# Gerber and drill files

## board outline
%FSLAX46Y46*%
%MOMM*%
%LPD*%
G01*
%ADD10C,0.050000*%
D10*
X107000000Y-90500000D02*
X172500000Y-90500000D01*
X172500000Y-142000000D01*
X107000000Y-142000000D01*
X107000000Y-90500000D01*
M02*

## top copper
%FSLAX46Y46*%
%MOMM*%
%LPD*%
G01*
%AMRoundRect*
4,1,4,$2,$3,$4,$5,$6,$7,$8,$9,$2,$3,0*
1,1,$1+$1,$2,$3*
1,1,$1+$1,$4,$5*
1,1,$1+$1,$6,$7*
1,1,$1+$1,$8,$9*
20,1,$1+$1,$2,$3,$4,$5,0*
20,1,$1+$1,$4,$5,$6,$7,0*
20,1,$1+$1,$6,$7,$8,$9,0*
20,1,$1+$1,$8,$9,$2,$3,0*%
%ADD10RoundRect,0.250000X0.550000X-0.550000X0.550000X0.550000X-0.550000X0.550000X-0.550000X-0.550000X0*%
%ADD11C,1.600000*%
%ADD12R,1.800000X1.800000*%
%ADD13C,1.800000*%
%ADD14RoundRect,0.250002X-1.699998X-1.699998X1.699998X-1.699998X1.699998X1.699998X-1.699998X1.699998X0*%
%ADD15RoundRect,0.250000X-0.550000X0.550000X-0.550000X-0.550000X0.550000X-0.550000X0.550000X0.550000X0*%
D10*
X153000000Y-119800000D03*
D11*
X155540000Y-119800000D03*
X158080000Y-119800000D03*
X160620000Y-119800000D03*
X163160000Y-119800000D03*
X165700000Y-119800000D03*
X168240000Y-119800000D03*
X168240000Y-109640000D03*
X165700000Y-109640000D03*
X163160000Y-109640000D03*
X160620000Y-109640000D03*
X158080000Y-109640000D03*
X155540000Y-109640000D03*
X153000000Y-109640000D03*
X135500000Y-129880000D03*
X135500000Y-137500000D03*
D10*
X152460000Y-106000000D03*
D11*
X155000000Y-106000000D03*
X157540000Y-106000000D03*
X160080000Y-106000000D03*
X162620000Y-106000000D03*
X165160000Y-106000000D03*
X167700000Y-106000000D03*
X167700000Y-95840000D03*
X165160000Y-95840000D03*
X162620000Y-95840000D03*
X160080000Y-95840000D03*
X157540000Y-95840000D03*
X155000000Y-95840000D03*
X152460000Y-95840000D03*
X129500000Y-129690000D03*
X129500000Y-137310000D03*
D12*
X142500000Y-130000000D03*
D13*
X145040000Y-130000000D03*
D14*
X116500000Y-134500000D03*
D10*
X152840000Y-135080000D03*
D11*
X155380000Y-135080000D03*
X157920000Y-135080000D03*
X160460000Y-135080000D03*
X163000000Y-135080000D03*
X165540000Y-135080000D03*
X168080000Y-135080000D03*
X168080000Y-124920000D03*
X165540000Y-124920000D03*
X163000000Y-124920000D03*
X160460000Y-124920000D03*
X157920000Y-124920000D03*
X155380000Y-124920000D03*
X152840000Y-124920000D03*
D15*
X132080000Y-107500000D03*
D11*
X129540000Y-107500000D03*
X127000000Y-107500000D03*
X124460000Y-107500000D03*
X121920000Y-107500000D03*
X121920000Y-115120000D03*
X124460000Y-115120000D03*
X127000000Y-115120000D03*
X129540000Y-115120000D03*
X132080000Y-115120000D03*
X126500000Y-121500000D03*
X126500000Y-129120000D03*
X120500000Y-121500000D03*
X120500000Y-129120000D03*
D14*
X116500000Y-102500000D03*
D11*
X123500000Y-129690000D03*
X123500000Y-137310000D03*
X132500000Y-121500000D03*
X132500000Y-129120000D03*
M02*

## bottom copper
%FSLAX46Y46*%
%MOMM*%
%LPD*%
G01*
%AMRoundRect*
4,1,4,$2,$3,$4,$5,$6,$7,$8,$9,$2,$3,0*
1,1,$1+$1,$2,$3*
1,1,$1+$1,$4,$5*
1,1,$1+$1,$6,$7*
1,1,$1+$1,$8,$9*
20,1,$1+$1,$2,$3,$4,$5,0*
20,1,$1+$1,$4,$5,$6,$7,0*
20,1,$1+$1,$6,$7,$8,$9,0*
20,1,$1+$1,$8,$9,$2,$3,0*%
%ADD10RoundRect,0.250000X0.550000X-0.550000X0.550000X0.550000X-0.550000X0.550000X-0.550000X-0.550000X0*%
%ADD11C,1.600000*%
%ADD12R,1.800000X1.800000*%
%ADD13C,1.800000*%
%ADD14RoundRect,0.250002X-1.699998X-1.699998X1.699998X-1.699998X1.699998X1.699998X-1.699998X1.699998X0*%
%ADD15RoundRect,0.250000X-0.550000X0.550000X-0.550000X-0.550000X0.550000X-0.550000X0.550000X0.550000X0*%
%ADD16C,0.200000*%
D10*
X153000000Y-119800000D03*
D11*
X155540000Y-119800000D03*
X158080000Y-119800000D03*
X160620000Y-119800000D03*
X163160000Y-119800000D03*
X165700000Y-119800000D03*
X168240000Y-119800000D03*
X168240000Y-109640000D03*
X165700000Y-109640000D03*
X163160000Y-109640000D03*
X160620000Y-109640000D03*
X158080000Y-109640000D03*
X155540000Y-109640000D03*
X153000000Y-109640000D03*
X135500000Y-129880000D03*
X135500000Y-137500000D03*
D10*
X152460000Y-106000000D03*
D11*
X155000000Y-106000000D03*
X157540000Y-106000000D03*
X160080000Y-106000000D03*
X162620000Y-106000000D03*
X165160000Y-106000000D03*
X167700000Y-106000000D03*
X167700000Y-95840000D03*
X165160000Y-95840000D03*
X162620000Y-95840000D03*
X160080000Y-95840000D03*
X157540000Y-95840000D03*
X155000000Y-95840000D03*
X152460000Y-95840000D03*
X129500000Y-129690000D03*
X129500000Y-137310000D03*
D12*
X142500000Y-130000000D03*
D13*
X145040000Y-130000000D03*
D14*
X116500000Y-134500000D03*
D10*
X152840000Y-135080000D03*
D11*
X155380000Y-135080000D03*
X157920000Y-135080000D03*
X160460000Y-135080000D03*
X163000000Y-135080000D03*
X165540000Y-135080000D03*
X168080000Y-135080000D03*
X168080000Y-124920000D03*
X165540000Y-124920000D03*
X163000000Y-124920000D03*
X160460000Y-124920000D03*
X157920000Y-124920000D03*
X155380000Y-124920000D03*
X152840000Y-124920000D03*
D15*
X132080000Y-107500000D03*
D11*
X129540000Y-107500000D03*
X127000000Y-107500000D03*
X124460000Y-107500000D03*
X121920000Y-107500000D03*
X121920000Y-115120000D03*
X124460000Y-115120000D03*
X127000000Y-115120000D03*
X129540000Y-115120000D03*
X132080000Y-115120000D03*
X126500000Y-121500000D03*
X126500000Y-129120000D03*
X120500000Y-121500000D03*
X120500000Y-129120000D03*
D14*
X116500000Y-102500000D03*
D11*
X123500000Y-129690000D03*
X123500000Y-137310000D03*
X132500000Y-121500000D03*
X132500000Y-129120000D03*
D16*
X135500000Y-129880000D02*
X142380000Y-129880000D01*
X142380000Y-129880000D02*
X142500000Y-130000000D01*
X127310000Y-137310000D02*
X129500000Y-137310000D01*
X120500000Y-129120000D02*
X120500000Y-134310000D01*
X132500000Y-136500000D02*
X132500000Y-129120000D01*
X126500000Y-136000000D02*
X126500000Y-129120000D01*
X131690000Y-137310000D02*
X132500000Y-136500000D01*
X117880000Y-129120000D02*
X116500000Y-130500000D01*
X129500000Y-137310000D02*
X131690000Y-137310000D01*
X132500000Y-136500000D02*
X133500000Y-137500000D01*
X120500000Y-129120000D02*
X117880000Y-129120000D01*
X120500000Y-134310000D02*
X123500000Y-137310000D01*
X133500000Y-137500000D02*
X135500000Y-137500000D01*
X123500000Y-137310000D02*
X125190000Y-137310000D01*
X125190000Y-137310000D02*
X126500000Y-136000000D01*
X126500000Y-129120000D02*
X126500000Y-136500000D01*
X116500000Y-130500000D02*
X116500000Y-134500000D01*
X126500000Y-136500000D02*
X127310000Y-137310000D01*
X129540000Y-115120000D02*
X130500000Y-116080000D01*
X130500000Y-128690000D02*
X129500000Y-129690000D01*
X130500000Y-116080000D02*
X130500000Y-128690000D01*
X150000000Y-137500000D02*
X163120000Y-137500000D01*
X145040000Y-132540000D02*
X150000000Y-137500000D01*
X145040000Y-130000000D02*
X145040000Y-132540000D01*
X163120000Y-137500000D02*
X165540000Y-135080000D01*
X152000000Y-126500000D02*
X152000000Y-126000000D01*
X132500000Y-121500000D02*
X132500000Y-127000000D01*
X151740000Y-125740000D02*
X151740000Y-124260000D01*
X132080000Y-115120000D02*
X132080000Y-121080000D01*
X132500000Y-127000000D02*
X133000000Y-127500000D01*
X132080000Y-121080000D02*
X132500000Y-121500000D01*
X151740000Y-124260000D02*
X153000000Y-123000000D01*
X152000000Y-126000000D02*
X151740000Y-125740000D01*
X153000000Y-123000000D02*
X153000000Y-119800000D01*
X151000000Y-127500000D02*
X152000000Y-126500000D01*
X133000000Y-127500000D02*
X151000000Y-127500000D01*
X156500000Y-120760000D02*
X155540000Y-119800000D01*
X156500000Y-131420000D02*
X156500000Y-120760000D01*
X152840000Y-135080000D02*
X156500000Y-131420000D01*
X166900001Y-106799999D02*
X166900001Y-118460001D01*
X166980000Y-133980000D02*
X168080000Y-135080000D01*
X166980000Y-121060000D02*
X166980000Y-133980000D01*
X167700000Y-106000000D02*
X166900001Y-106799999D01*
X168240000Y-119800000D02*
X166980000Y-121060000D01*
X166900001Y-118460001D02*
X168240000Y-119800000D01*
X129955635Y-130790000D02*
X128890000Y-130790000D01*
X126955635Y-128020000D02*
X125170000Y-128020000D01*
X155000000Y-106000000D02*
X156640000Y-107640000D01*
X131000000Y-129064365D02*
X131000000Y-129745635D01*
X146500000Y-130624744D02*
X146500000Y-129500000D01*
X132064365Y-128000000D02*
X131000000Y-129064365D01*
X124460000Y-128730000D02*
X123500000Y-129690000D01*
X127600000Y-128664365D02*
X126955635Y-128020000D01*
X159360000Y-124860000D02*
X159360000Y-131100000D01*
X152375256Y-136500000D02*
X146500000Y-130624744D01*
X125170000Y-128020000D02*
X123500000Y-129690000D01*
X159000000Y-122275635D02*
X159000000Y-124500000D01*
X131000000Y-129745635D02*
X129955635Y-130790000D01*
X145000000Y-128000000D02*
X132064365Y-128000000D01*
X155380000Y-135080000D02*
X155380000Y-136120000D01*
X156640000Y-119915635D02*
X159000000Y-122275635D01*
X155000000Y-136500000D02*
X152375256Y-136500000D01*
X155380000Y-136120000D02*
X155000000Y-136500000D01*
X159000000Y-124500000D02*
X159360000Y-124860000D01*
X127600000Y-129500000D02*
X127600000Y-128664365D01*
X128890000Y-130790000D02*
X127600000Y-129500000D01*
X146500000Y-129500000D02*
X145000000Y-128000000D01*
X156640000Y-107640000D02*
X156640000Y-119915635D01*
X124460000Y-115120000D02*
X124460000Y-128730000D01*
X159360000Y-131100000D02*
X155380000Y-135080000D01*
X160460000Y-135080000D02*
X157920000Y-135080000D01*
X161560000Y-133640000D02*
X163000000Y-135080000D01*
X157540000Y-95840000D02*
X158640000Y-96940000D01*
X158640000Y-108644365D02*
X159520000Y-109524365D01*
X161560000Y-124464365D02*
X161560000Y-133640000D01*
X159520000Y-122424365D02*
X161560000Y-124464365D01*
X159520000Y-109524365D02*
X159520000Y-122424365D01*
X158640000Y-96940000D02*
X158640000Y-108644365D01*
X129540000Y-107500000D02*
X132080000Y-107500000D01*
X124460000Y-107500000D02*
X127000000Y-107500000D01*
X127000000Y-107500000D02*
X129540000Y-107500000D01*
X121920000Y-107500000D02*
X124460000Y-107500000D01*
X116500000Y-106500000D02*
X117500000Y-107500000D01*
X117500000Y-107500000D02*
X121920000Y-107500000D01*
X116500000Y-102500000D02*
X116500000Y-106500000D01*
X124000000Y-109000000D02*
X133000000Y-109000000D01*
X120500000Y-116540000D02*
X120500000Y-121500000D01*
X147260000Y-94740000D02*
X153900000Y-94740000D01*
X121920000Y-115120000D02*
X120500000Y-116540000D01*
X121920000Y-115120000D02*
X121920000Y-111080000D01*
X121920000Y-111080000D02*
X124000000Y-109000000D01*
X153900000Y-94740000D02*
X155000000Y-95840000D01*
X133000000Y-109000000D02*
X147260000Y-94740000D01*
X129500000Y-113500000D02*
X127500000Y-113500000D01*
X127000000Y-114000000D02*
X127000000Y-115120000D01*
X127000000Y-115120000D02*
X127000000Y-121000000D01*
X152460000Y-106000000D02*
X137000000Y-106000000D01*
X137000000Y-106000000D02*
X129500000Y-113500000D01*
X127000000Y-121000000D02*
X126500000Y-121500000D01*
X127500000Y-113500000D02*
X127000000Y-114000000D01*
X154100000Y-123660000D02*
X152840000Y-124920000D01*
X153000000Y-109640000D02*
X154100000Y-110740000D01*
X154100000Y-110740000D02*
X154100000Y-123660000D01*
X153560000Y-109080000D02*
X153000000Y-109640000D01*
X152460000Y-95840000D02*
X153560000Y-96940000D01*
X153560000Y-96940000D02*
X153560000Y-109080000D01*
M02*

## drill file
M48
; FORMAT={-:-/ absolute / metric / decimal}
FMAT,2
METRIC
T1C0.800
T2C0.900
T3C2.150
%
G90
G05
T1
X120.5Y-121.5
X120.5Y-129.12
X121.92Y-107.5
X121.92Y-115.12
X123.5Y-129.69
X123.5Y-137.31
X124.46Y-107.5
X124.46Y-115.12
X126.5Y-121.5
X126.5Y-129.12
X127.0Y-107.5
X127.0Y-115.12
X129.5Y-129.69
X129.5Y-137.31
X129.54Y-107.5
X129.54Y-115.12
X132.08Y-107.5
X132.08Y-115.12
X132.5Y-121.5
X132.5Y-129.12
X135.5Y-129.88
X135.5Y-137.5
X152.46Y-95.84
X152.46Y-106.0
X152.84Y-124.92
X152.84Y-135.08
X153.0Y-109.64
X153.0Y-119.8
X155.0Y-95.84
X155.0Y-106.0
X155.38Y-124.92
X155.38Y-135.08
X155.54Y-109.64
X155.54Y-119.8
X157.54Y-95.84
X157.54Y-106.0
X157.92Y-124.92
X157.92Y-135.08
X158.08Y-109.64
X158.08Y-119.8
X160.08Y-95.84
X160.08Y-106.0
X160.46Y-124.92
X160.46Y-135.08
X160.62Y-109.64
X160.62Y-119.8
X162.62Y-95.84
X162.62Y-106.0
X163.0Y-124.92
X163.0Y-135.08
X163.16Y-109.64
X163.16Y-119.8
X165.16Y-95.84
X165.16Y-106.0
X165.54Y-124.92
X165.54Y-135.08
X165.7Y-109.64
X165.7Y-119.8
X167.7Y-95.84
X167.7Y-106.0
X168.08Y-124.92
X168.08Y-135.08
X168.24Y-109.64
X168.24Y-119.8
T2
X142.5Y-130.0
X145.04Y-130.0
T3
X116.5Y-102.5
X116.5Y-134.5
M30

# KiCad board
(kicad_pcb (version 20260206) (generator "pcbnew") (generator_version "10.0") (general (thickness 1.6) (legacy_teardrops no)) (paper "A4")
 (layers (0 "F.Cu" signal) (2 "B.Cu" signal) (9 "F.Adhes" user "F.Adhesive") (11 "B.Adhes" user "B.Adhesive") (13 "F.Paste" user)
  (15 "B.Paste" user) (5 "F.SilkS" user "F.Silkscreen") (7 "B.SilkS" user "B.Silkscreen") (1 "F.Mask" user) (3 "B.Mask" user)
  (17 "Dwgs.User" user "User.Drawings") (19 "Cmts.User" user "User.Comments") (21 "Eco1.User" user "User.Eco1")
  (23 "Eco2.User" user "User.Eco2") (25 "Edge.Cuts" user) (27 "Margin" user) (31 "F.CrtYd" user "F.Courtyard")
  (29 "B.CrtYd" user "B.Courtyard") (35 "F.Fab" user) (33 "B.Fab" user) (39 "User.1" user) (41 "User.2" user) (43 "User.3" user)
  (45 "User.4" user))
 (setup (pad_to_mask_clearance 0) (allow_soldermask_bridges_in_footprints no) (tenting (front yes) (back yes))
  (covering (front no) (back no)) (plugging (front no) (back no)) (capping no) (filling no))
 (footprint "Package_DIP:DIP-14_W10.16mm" (layer "F.Cu") (at 153 119.8 90)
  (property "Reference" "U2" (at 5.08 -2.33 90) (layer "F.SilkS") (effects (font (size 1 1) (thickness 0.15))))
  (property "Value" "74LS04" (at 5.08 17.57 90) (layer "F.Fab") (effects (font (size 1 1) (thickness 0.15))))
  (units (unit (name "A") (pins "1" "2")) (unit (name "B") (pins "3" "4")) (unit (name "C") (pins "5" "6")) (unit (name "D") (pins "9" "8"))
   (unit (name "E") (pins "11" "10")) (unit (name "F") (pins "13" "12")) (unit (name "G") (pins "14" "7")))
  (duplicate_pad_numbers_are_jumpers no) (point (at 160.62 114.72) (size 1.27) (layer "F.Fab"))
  (pad "1" thru_hole roundrect (at 0 0 90) (size 1.6 1.6) (drill 0.8) (layers "*.Cu" "*.Mask") (remove_unused_layers no)
   (roundrect_rratio 0.15625) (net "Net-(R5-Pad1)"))
  (pad "2" thru_hole circle (at 0 2.54 90) (size 1.6 1.6) (drill 0.8) (layers "*.Cu" "*.Mask") (remove_unused_layers no)
   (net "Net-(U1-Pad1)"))
  (pad "3" thru_hole circle (at 0 5.08 90) (size 1.6 1.6) (drill 0.8) (layers "*.Cu" "*.Mask") (remove_unused_layers no)
   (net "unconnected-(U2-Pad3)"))
  (pad "4" thru_hole circle (at 0 7.62 90) (size 1.6 1.6) (drill 0.8) (layers "*.Cu" "*.Mask") (remove_unused_layers no)
   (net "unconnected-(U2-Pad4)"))
  (pad "5" thru_hole circle (at 0 10.16 90) (size 1.6 1.6) (drill 0.8) (layers "*.Cu" "*.Mask") (remove_unused_layers no)
   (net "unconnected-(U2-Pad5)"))
  (pad "6" thru_hole circle (at 0 12.7 90) (size 1.6 1.6) (drill 0.8) (layers "*.Cu" "*.Mask") (remove_unused_layers no)
   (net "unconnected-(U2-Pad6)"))
  (pad "7" thru_hole circle (at 0 15.24 90) (size 1.6 1.6) (drill 0.8) (layers "*.Cu" "*.Mask") (remove_unused_layers no)
   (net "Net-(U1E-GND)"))
  (pad "8" thru_hole circle (at 10.16 15.24 90) (size 1.6 1.6) (drill 0.8) (layers "*.Cu" "*.Mask") (remove_unused_layers no)
   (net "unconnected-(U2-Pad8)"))
  (pad "9" thru_hole circle (at 10.16 12.7 90) (size 1.6 1.6) (drill 0.8) (layers "*.Cu" "*.Mask") (remove_unused_layers no)
   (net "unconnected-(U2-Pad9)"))
  (pad "10" thru_hole circle (at 10.16 10.16 90) (size 1.6 1.6) (drill 0.8) (layers "*.Cu" "*.Mask") (remove_unused_layers no)
   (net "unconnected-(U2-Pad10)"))
  (pad "11" thru_hole circle (at 10.16 7.62 90) (size 1.6 1.6) (drill 0.8) (layers "*.Cu" "*.Mask") (remove_unused_layers no)
   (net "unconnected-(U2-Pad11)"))
  (pad "12" thru_hole circle (at 10.16 5.08 90) (size 1.6 1.6) (drill 0.8) (layers "*.Cu" "*.Mask") (remove_unused_layers no)
   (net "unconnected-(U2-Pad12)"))
  (pad "13" thru_hole circle (at 10.16 2.54 90) (size 1.6 1.6) (drill 0.8) (layers "*.Cu" "*.Mask") (remove_unused_layers no)
   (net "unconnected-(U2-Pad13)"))
  (pad "14" thru_hole circle (at 10.16 0 90) (size 1.6 1.6) (drill 0.8) (layers "*.Cu" "*.Mask") (remove_unused_layers no)
   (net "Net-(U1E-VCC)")))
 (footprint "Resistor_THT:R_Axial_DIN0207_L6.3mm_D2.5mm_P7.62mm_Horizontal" (layer "F.Cu") (at 135.5 129.88 -90)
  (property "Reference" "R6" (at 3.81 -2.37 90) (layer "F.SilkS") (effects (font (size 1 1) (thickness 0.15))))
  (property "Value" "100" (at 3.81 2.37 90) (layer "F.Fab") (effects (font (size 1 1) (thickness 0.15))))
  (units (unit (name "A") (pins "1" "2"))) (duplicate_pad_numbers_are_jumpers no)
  (pad "1" thru_hole circle (at 0 0 270) (size 1.6 1.6) (drill 0.8) (layers "*.Cu" "*.Mask") (remove_unused_layers no) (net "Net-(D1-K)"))
  (pad "2" thru_hole circle (at 7.62 0 270) (size 1.6 1.6) (drill 0.8) (layers "*.Cu" "*.Mask") (remove_unused_layers no) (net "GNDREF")))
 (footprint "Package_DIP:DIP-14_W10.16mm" (layer "F.Cu") (at 152.46 106 90)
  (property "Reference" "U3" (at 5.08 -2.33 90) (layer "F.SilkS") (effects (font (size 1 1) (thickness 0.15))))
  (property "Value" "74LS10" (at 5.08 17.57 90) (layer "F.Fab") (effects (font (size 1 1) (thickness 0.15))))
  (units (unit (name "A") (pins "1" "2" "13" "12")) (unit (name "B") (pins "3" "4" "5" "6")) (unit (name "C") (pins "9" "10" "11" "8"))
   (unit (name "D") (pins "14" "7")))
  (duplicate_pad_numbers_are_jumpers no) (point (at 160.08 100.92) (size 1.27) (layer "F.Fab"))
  (pad "1" thru_hole roundrect (at 0 0 90) (size 1.6 1.6) (drill 0.8) (layers "*.Cu" "*.Mask") (remove_unused_layers no)
   (roundrect_rratio 0.15625) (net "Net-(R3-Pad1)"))
  (pad "2" thru_hole circle (at 0 2.54 90) (size 1.6 1.6) (drill 0.8) (layers "*.Cu" "*.Mask") (remove_unused_layers no)
   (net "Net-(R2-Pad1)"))
  (pad "3" thru_hole circle (at 0 5.08 90) (size 1.6 1.6) (drill 0.8) (layers "*.Cu" "*.Mask") (remove_unused_layers no)
   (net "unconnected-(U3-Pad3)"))
  (pad "4" thru_hole circle (at 0 7.62 90) (size 1.6 1.6) (drill 0.8) (layers "*.Cu" "*.Mask") (remove_unused_layers no)
   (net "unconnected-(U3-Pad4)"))
  (pad "5" thru_hole circle (at 0 10.16 90) (size 1.6 1.6) (drill 0.8) (layers "*.Cu" "*.Mask") (remove_unused_layers no)
   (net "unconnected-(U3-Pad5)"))
  (pad "6" thru_hole circle (at 0 12.7 90) (size 1.6 1.6) (drill 0.8) (layers "*.Cu" "*.Mask") (remove_unused_layers no)
   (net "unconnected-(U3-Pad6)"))
  (pad "7" thru_hole circle (at 0 15.24 90) (size 1.6 1.6) (drill 0.8) (layers "*.Cu" "*.Mask") (remove_unused_layers no)
   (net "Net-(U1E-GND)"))
  (pad "8" thru_hole circle (at 10.16 15.24 90) (size 1.6 1.6) (drill 0.8) (layers "*.Cu" "*.Mask") (remove_unused_layers no)
   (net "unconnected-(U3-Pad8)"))
  (pad "9" thru_hole circle (at 10.16 12.7 90) (size 1.6 1.6) (drill 0.8) (layers "*.Cu" "*.Mask") (remove_unused_layers no)
   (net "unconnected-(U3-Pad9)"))
  (pad "10" thru_hole circle (at 10.16 10.16 90) (size 1.6 1.6) (drill 0.8) (layers "*.Cu" "*.Mask") (remove_unused_layers no)
   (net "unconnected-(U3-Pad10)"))
  (pad "11" thru_hole circle (at 10.16 7.62 90) (size 1.6 1.6) (drill 0.8) (layers "*.Cu" "*.Mask") (remove_unused_layers no)
   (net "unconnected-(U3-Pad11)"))
  (pad "12" thru_hole circle (at 10.16 5.08 90) (size 1.6 1.6) (drill 0.8) (layers "*.Cu" "*.Mask") (remove_unused_layers no)
   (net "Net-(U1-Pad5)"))
  (pad "13" thru_hole circle (at 10.16 2.54 90) (size 1.6 1.6) (drill 0.8) (layers "*.Cu" "*.Mask") (remove_unused_layers no)
   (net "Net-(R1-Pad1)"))
  (pad "14" thru_hole circle (at 10.16 0 90) (size 1.6 1.6) (drill 0.8) (layers "*.Cu" "*.Mask") (remove_unused_layers no)
   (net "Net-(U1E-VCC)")))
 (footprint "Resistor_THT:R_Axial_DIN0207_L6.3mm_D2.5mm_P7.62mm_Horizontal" (layer "F.Cu") (at 129.5 129.69 -90)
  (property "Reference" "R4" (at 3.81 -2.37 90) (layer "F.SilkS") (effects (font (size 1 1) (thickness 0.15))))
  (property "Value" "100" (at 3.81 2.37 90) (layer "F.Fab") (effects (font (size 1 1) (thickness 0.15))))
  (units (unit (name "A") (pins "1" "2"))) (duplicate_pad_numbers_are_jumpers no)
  (pad "1" thru_hole circle (at 0 0 270) (size 1.6 1.6) (drill 0.8) (layers "*.Cu" "*.Mask") (remove_unused_layers no) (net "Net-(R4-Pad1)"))
  (pad "2" thru_hole circle (at 7.62 0 270) (size 1.6 1.6) (drill 0.8) (layers "*.Cu" "*.Mask") (remove_unused_layers no) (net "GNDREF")))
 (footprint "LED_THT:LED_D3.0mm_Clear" (layer "F.Cu") (at 142.5 130)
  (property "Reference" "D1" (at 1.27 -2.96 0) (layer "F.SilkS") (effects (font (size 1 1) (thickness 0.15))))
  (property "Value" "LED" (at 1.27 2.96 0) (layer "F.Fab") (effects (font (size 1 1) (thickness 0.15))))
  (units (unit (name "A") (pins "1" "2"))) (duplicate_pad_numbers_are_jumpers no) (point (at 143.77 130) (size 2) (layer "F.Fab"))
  (pad "1" thru_hole rect (at 0 0) (size 1.8 1.8) (drill 0.9) (layers "*.Cu" "*.Mask") (remove_unused_layers no) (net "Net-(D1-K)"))
  (pad "2" thru_hole circle (at 2.54 0) (size 1.8 1.8) (drill 0.9) (layers "*.Cu" "*.Mask") (remove_unused_layers no) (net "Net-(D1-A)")))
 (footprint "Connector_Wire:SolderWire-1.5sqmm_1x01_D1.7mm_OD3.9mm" (layer "F.Cu") (at 116.5 134.5)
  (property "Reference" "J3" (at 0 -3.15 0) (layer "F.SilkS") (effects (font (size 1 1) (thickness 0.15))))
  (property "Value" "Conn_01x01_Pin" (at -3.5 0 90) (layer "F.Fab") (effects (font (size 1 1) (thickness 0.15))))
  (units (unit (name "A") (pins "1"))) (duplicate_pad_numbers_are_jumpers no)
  (pad "1" thru_hole roundrect (at 0 0) (size 3.9 3.9) (drill 2.15) (layers "*.Cu" "*.Mask") (remove_unused_layers no)
   (roundrect_rratio 0.064103) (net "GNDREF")))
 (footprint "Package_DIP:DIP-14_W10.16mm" (layer "F.Cu") (at 152.84 135.08 90)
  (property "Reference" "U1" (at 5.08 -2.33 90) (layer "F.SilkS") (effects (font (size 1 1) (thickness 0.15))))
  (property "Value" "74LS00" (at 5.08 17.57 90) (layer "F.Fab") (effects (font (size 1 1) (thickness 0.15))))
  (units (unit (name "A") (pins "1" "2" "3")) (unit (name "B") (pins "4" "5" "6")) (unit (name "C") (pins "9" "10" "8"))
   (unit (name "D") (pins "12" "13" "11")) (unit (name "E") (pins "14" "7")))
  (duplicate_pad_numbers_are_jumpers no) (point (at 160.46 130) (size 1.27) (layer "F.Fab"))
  (pad "1" thru_hole roundrect (at 0 0 90) (size 1.6 1.6) (drill 0.8) (layers "*.Cu" "*.Mask") (remove_unused_layers no)
   (roundrect_rratio 0.15625) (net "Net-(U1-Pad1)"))
  (pad "2" thru_hole circle (at 0 2.54 90) (size 1.6 1.6) (drill 0.8) (layers "*.Cu" "*.Mask") (remove_unused_layers no)
   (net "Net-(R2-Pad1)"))
  (pad "3" thru_hole circle (at 0 5.08 90) (size 1.6 1.6) (drill 0.8) (layers "*.Cu" "*.Mask") (remove_unused_layers no)
   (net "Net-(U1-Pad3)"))
  (pad "4" thru_hole circle (at 0 7.62 90) (size 1.6 1.6) (drill 0.8) (layers "*.Cu" "*.Mask") (remove_unused_layers no)
   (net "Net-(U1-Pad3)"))
  (pad "5" thru_hole circle (at 0 10.16 90) (size 1.6 1.6) (drill 0.8) (layers "*.Cu" "*.Mask") (remove_unused_layers no)
   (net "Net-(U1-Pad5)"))
  (pad "6" thru_hole circle (at 0 12.7 90) (size 1.6 1.6) (drill 0.8) (layers "*.Cu" "*.Mask") (remove_unused_layers no) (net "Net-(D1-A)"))
  (pad "7" thru_hole circle (at 0 15.24 90) (size 1.6 1.6) (drill 0.8) (layers "*.Cu" "*.Mask") (remove_unused_layers no)
   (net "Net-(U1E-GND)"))
  (pad "8" thru_hole circle (at 10.16 15.24 90) (size 1.6 1.6) (drill 0.8) (layers "*.Cu" "*.Mask") (remove_unused_layers no)
   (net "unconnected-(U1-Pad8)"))
  (pad "9" thru_hole circle (at 10.16 12.7 90) (size 1.6 1.6) (drill 0.8) (layers "*.Cu" "*.Mask") (remove_unused_layers no)
   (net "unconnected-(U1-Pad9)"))
  (pad "10" thru_hole circle (at 10.16 10.16 90) (size 1.6 1.6) (drill 0.8) (layers "*.Cu" "*.Mask") (remove_unused_layers no)
   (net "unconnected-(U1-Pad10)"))
  (pad "11" thru_hole circle (at 10.16 7.62 90) (size 1.6 1.6) (drill 0.8) (layers "*.Cu" "*.Mask") (remove_unused_layers no)
   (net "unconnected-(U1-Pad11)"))
  (pad "12" thru_hole circle (at 10.16 5.08 90) (size 1.6 1.6) (drill 0.8) (layers "*.Cu" "*.Mask") (remove_unused_layers no)
   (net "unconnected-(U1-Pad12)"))
  (pad "13" thru_hole circle (at 10.16 2.54 90) (size 1.6 1.6) (drill 0.8) (layers "*.Cu" "*.Mask") (remove_unused_layers no)
   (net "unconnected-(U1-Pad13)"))
  (pad "14" thru_hole circle (at 10.16 0 90) (size 1.6 1.6) (drill 0.8) (layers "*.Cu" "*.Mask") (remove_unused_layers no)
   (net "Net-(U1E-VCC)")))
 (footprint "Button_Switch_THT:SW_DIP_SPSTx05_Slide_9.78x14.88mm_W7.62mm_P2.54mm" (layer "F.Cu") (at 132.08 107.5 -90)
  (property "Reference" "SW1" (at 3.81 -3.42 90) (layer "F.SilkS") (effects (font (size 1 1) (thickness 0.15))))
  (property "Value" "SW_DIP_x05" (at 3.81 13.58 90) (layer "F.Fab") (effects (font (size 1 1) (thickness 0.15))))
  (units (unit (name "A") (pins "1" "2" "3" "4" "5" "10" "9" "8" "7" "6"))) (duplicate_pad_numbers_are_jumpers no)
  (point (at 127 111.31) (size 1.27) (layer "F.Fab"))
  (pad "1" thru_hole roundrect (at 0 0 270) (size 1.6 1.6) (drill 0.8) (layers "*.Cu" "*.Mask") (remove_unused_layers no)
   (roundrect_rratio 0.15625) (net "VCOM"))
  (pad "2" thru_hole circle (at 0 2.54 270) (size 1.6 1.6) (drill 0.8) (layers "*.Cu" "*.Mask") (remove_unused_layers no) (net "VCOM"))
  (pad "3" thru_hole circle (at 0 5.08 270) (size 1.6 1.6) (drill 0.8) (layers "*.Cu" "*.Mask") (remove_unused_layers no) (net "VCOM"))
  (pad "4" thru_hole circle (at 0 7.62 270) (size 1.6 1.6) (drill 0.8) (layers "*.Cu" "*.Mask") (remove_unused_layers no) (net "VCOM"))
  (pad "5" thru_hole circle (at 0 10.16 270) (size 1.6 1.6) (drill 0.8) (layers "*.Cu" "*.Mask") (remove_unused_layers no) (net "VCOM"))
  (pad "6" thru_hole circle (at 7.62 10.16 270) (size 1.6 1.6) (drill 0.8) (layers "*.Cu" "*.Mask") (remove_unused_layers no)
   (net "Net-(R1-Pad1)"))
  (pad "7" thru_hole circle (at 7.62 7.62 270) (size 1.6 1.6) (drill 0.8) (layers "*.Cu" "*.Mask") (remove_unused_layers no)
   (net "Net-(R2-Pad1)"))
  (pad "8" thru_hole circle (at 7.62 5.08 270) (size 1.6 1.6) (drill 0.8) (layers "*.Cu" "*.Mask") (remove_unused_layers no)
   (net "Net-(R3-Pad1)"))
  (pad "9" thru_hole circle (at 7.62 2.54 270) (size 1.6 1.6) (drill 0.8) (layers "*.Cu" "*.Mask") (remove_unused_layers no)
   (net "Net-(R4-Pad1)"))
  (pad "10" thru_hole circle (at 7.62 0 270) (size 1.6 1.6) (drill 0.8) (layers "*.Cu" "*.Mask") (remove_unused_layers no)
   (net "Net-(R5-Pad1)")))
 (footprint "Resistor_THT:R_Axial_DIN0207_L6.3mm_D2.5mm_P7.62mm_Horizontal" (layer "F.Cu") (at 126.5 121.5 -90)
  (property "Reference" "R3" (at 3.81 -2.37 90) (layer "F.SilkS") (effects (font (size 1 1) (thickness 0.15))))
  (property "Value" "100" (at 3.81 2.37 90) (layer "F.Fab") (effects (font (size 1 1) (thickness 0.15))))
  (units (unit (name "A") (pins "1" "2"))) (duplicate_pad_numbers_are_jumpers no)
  (pad "1" thru_hole circle (at 0 0 270) (size 1.6 1.6) (drill 0.8) (layers "*.Cu" "*.Mask") (remove_unused_layers no) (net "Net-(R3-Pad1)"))
  (pad "2" thru_hole circle (at 7.62 0 270) (size 1.6 1.6) (drill 0.8) (layers "*.Cu" "*.Mask") (remove_unused_layers no) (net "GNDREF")))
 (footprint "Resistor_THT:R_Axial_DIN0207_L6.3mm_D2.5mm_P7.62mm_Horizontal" (layer "F.Cu") (at 120.5 121.5 -90)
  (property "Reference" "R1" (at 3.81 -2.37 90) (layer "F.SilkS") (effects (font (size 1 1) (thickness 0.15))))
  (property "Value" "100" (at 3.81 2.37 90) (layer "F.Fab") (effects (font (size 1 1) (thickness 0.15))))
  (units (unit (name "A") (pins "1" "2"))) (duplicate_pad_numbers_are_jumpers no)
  (pad "1" thru_hole circle (at 0 0 270) (size 1.6 1.6) (drill 0.8) (layers "*.Cu" "*.Mask") (remove_unused_layers no) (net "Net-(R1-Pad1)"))
  (pad "2" thru_hole circle (at 7.62 0 270) (size 1.6 1.6) (drill 0.8) (layers "*.Cu" "*.Mask") (remove_unused_layers no) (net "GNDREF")))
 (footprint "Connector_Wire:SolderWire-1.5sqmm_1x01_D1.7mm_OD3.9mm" (layer "F.Cu") (at 116.5 102.5)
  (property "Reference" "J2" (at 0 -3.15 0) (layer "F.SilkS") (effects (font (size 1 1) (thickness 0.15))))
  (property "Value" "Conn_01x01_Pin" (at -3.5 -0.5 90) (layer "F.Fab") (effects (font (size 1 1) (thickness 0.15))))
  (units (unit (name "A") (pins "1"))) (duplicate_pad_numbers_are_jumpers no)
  (pad "1" thru_hole roundrect (at 0 0) (size 3.9 3.9) (drill 2.15) (layers "*.Cu" "*.Mask") (remove_unused_layers no)
   (roundrect_rratio 0.064103) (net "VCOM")))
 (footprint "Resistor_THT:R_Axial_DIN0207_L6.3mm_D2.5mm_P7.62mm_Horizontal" (layer "F.Cu") (at 123.5 129.69 -90)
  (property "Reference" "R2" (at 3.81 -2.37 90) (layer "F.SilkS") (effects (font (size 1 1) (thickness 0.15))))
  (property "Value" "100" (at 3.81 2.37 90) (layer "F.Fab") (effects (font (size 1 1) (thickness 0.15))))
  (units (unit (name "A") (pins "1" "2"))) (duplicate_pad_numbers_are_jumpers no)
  (pad "1" thru_hole circle (at 0 0 270) (size 1.6 1.6) (drill 0.8) (layers "*.Cu" "*.Mask") (remove_unused_layers no) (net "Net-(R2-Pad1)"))
  (pad "2" thru_hole circle (at 7.62 0 270) (size 1.6 1.6) (drill 0.8) (layers "*.Cu" "*.Mask") (remove_unused_layers no) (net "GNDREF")))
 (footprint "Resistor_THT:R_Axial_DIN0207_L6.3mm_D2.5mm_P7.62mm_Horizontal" (layer "F.Cu") (at 132.5 121.5 -90)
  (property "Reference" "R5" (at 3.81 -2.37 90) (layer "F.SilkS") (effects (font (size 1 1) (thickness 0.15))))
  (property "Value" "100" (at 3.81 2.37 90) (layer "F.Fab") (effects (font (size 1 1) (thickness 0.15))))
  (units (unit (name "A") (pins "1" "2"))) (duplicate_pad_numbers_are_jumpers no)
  (pad "1" thru_hole circle (at 0 0 270) (size 1.6 1.6) (drill 0.8) (layers "*.Cu" "*.Mask") (remove_unused_layers no) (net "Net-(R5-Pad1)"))
  (pad "2" thru_hole circle (at 7.62 0 270) (size 1.6 1.6) (drill 0.8) (layers "*.Cu" "*.Mask") (remove_unused_layers no) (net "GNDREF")))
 (gr_rect (start 107 90.5) (end 172.5 142) (stroke (width 0.05) (type default)) (fill no) (layer "Edge.Cuts"))
 (segment (start 135.5 129.88) (end 142.38 129.88) (width 0.2) (layer "B.Cu") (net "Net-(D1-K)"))
 (segment (start 142.38 129.88) (end 142.5 130) (width 0.2) (layer "B.Cu") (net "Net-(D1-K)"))
 (segment (start 127.31 137.31) (end 129.5 137.31) (width 0.2) (layer "B.Cu") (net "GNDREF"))
 (segment (start 120.5 129.12) (end 120.5 134.31) (width 0.2) (layer "B.Cu") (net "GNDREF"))
 (segment (start 132.5 136.5) (end 132.5 129.12) (width 0.2) (layer "B.Cu") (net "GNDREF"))
 (segment (start 126.5 136) (end 126.5 129.12) (width 0.2) (layer "B.Cu") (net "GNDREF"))
 (segment (start 131.69 137.31) (end 132.5 136.5) (width 0.2) (layer "B.Cu") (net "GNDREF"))
 (segment (start 117.88 129.12) (end 116.5 130.5) (width 0.2) (layer "B.Cu") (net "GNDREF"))
 (segment (start 129.5 137.31) (end 131.69 137.31) (width 0.2) (layer "B.Cu") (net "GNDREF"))
 (segment (start 132.5 136.5) (end 133.5 137.5) (width 0.2) (layer "B.Cu") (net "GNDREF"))
 (segment (start 120.5 129.12) (end 117.88 129.12) (width 0.2) (layer "B.Cu") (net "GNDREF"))
 (segment (start 120.5 134.31) (end 123.5 137.31) (width 0.2) (layer "B.Cu") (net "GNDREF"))
 (segment (start 133.5 137.5) (end 135.5 137.5) (width 0.2) (layer "B.Cu") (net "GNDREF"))
 (segment (start 123.5 137.31) (end 125.19 137.31) (width 0.2) (layer "B.Cu") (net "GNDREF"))
 (segment (start 125.19 137.31) (end 126.5 136) (width 0.2) (layer "B.Cu") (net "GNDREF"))
 (segment (start 126.5 129.12) (end 126.5 136.5) (width 0.2) (layer "B.Cu") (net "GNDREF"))
 (segment (start 116.5 130.5) (end 116.5 134.5) (width 0.2) (layer "B.Cu") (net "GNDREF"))
 (segment (start 126.5 136.5) (end 127.31 137.31) (width 0.2) (layer "B.Cu") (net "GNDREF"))
 (segment (start 129.54 115.12) (end 130.5 116.08) (width 0.2) (layer "B.Cu") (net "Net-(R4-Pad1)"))
 (segment (start 130.5 128.69) (end 129.5 129.69) (width 0.2) (layer "B.Cu") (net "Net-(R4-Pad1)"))
 (segment (start 130.5 116.08) (end 130.5 128.69) (width 0.2) (layer "B.Cu") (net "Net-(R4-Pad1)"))
 (segment (start 150 137.5) (end 163.12 137.5) (width 0.2) (layer "B.Cu") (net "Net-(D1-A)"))
 (segment (start 145.04 132.54) (end 150 137.5) (width 0.2) (layer "B.Cu") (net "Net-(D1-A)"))
 (segment (start 145.04 130) (end 145.04 132.54) (width 0.2) (layer "B.Cu") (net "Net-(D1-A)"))
 (segment (start 163.12 137.5) (end 165.54 135.08) (width 0.2) (layer "B.Cu") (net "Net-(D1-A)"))
 (segment (start 152 126.5) (end 152 126) (width 0.2) (layer "B.Cu") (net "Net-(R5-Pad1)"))
 (segment (start 132.5 121.5) (end 132.5 127) (width 0.2) (layer "B.Cu") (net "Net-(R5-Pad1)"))
 (segment (start 151.74 125.74) (end 151.74 124.26) (width 0.2) (layer "B.Cu") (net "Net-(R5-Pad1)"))
 (segment (start 132.08 115.12) (end 132.08 121.08) (width 0.2) (layer "B.Cu") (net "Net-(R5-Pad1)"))
 (segment (start 132.5 127) (end 133 127.5) (width 0.2) (layer "B.Cu") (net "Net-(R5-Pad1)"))
 (segment (start 132.08 121.08) (end 132.5 121.5) (width 0.2) (layer "B.Cu") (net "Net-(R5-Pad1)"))
 (segment (start 151.74 124.26) (end 153 123) (width 0.2) (layer "B.Cu") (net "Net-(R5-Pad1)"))
 (segment (start 152 126) (end 151.74 125.74) (width 0.2) (layer "B.Cu") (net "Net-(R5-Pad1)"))
 (segment (start 153 123) (end 153 119.8) (width 0.2) (layer "B.Cu") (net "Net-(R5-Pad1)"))
 (segment (start 151 127.5) (end 152 126.5) (width 0.2) (layer "B.Cu") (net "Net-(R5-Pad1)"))
 (segment (start 133 127.5) (end 151 127.5) (width 0.2) (layer "B.Cu") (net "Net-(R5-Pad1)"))
 (segment (start 156.5 120.76) (end 155.54 119.8) (width 0.2) (layer "B.Cu") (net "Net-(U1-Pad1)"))
 (segment (start 156.5 131.42) (end 156.5 120.76) (width 0.2) (layer "B.Cu") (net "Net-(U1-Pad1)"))
 (segment (start 152.84 135.08) (end 156.5 131.42) (width 0.2) (layer "B.Cu") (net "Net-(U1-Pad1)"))
 (segment (start 166.900001 106.799999) (end 166.900001 118.460001) (width 0.2) (layer "B.Cu") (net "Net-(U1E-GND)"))
 (segment (start 166.98 133.98) (end 168.08 135.08) (width 0.2) (layer "B.Cu") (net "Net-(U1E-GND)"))
 (segment (start 166.98 121.06) (end 166.98 133.98) (width 0.2) (layer "B.Cu") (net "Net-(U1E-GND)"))
 (segment (start 167.7 106) (end 166.900001 106.799999) (width 0.2) (layer "B.Cu") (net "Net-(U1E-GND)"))
 (segment (start 168.24 119.8) (end 166.98 121.06) (width 0.2) (layer "B.Cu") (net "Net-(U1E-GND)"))
 (segment (start 166.900001 118.460001) (end 168.24 119.8) (width 0.2) (layer "B.Cu") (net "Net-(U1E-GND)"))
 (segment (start 129.955635 130.79) (end 128.89 130.79) (width 0.2) (layer "B.Cu") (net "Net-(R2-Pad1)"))
 (segment (start 126.955635 128.02) (end 125.17 128.02) (width 0.2) (layer "B.Cu") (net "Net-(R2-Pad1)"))
 (segment (start 155 106) (end 156.64 107.64) (width 0.2) (layer "B.Cu") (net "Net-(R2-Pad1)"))
 (segment (start 131 129.064365) (end 131 129.745635) (width 0.2) (layer "B.Cu") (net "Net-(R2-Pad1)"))
 (segment (start 146.5 130.624744) (end 146.5 129.5) (width 0.2) (layer "B.Cu") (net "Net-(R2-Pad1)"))
 (segment (start 132.064365 128) (end 131 129.064365) (width 0.2) (layer "B.Cu") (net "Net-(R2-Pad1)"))
 (segment (start 124.46 128.73) (end 123.5 129.69) (width 0.2) (layer "B.Cu") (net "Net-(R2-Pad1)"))
 (segment (start 127.6 128.664365) (end 126.955635 128.02) (width 0.2) (layer "B.Cu") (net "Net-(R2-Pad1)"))
 (segment (start 159.36 124.86) (end 159.36 131.1) (width 0.2) (layer "B.Cu") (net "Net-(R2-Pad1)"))
 (segment (start 152.375256 136.5) (end 146.5 130.624744) (width 0.2) (layer "B.Cu") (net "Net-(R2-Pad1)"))
 (segment (start 125.17 128.02) (end 123.5 129.69) (width 0.2) (layer "B.Cu") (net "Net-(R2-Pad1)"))
 (segment (start 159 122.275635) (end 159 124.5) (width 0.2) (layer "B.Cu") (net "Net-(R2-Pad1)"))
 (segment (start 131 129.745635) (end 129.955635 130.79) (width 0.2) (layer "B.Cu") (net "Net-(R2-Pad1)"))
 (segment (start 145 128) (end 132.064365 128) (width 0.2) (layer "B.Cu") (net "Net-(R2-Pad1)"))
 (segment (start 155.38 135.08) (end 155.38 136.12) (width 0.2) (layer "B.Cu") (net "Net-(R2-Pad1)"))
 (segment (start 156.64 119.915635) (end 159 122.275635) (width 0.2) (layer "B.Cu") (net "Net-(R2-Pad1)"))
 (segment (start 155 136.5) (end 152.375256 136.5) (width 0.2) (layer "B.Cu") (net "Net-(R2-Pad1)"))
 (segment (start 155.38 136.12) (end 155 136.5) (width 0.2) (layer "B.Cu") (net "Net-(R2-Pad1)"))
 (segment (start 159 124.5) (end 159.36 124.86) (width 0.2) (layer "B.Cu") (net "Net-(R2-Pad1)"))
 (segment (start 127.6 129.5) (end 127.6 128.664365) (width 0.2) (layer "B.Cu") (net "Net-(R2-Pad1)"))
 (segment (start 128.89 130.79) (end 127.6 129.5) (width 0.2) (layer "B.Cu") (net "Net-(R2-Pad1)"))
 (segment (start 146.5 129.5) (end 145 128) (width 0.2) (layer "B.Cu") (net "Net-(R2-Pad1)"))
 (segment (start 156.64 107.64) (end 156.64 119.915635) (width 0.2) (layer "B.Cu") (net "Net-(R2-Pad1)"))
 (segment (start 124.46 115.12) (end 124.46 128.73) (width 0.2) (layer "B.Cu") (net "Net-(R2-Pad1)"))
 (segment (start 159.36 131.1) (end 155.38 135.08) (width 0.2) (layer "B.Cu") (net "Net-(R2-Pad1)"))
 (segment (start 160.46 135.08) (end 157.92 135.08) (width 0.2) (layer "B.Cu") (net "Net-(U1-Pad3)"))
 (segment (start 161.56 133.64) (end 163 135.08) (width 0.2) (layer "B.Cu") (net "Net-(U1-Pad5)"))
 (segment (start 157.54 95.84) (end 158.64 96.94) (width 0.2) (layer "B.Cu") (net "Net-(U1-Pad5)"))
 (segment (start 158.64 108.644365) (end 159.52 109.524365) (width 0.2) (layer "B.Cu") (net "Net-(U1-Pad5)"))
 (segment (start 161.56 124.464365) (end 161.56 133.64) (width 0.2) (layer "B.Cu") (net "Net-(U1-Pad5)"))
 (segment (start 159.52 122.424365) (end 161.56 124.464365) (width 0.2) (layer "B.Cu") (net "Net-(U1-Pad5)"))
 (segment (start 159.52 109.524365) (end 159.52 122.424365) (width 0.2) (layer "B.Cu") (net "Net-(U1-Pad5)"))
 (segment (start 158.64 96.94) (end 158.64 108.644365) (width 0.2) (layer "B.Cu") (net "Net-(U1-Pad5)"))
 (segment (start 129.54 107.5) (end 132.08 107.5) (width 0.2) (layer "B.Cu") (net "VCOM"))
 (segment (start 124.46 107.5) (end 127 107.5) (width 0.2) (layer "B.Cu") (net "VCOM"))
 (segment (start 127 107.5) (end 129.54 107.5) (width 0.2) (layer "B.Cu") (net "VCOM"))
 (segment (start 121.92 107.5) (end 124.46 107.5) (width 0.2) (layer "B.Cu") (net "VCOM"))
 (segment (start 116.5 106.5) (end 117.5 107.5) (width 0.2) (layer "B.Cu") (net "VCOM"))
 (segment (start 117.5 107.5) (end 121.92 107.5) (width 0.2) (layer "B.Cu") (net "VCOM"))
 (segment (start 116.5 102.5) (end 116.5 106.5) (width 0.2) (layer "B.Cu") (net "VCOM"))
 (segment (start 124 109) (end 133 109) (width 0.2) (layer "B.Cu") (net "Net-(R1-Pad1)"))
 (segment (start 120.5 116.54) (end 120.5 121.5) (width 0.2) (layer "B.Cu") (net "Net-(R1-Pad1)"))
 (segment (start 147.26 94.74) (end 153.9 94.74) (width 0.2) (layer "B.Cu") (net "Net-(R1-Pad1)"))
 (segment (start 121.92 115.12) (end 120.5 116.54) (width 0.2) (layer "B.Cu") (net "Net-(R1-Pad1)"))
 (segment (start 121.92 115.12) (end 121.92 111.08) (width 0.2) (layer "B.Cu") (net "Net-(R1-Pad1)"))
 (segment (start 121.92 111.08) (end 124 109) (width 0.2) (layer "B.Cu") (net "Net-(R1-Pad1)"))
 (segment (start 153.9 94.74) (end 155 95.84) (width 0.2) (layer "B.Cu") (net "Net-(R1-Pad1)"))
 (segment (start 133 109) (end 147.26 94.74) (width 0.2) (layer "B.Cu") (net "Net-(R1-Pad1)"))
 (segment (start 129.5 113.5) (end 127.5 113.5) (width 0.2) (layer "B.Cu") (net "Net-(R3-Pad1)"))
 (segment (start 127 114) (end 127 115.12) (width 0.2) (layer "B.Cu") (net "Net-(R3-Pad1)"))
 (segment (start 127 115.12) (end 127 121) (width 0.2) (layer "B.Cu") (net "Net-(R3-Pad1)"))
 (segment (start 152.46 106) (end 137 106) (width 0.2) (layer "B.Cu") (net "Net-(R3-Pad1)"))
 (segment (start 137 106) (end 129.5 113.5) (width 0.2) (layer "B.Cu") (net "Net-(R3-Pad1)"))
 (segment (start 127 121) (end 126.5 121.5) (width 0.2) (layer "B.Cu") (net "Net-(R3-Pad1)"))
 (segment (start 127.5 113.5) (end 127 114) (width 0.2) (layer "B.Cu") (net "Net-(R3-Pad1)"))
 (segment (start 154.1 123.66) (end 152.84 124.92) (width 0.2) (layer "B.Cu") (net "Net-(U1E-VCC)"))
 (segment (start 153 109.64) (end 154.1 110.74) (width 0.2) (layer "B.Cu") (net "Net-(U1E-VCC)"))
 (segment (start 154.1 110.74) (end 154.1 123.66) (width 0.2) (layer "B.Cu") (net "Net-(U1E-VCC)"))
 (segment (start 153.56 109.08) (end 153 109.64) (width 0.2) (layer "B.Cu") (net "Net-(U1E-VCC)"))
 (segment (start 152.46 95.84) (end 153.56 96.94) (width 0.2) (layer "B.Cu") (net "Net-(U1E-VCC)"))
 (segment (start 153.56 96.94) (end 153.56 109.08) (width 0.2) (layer "B.Cu") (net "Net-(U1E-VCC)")))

